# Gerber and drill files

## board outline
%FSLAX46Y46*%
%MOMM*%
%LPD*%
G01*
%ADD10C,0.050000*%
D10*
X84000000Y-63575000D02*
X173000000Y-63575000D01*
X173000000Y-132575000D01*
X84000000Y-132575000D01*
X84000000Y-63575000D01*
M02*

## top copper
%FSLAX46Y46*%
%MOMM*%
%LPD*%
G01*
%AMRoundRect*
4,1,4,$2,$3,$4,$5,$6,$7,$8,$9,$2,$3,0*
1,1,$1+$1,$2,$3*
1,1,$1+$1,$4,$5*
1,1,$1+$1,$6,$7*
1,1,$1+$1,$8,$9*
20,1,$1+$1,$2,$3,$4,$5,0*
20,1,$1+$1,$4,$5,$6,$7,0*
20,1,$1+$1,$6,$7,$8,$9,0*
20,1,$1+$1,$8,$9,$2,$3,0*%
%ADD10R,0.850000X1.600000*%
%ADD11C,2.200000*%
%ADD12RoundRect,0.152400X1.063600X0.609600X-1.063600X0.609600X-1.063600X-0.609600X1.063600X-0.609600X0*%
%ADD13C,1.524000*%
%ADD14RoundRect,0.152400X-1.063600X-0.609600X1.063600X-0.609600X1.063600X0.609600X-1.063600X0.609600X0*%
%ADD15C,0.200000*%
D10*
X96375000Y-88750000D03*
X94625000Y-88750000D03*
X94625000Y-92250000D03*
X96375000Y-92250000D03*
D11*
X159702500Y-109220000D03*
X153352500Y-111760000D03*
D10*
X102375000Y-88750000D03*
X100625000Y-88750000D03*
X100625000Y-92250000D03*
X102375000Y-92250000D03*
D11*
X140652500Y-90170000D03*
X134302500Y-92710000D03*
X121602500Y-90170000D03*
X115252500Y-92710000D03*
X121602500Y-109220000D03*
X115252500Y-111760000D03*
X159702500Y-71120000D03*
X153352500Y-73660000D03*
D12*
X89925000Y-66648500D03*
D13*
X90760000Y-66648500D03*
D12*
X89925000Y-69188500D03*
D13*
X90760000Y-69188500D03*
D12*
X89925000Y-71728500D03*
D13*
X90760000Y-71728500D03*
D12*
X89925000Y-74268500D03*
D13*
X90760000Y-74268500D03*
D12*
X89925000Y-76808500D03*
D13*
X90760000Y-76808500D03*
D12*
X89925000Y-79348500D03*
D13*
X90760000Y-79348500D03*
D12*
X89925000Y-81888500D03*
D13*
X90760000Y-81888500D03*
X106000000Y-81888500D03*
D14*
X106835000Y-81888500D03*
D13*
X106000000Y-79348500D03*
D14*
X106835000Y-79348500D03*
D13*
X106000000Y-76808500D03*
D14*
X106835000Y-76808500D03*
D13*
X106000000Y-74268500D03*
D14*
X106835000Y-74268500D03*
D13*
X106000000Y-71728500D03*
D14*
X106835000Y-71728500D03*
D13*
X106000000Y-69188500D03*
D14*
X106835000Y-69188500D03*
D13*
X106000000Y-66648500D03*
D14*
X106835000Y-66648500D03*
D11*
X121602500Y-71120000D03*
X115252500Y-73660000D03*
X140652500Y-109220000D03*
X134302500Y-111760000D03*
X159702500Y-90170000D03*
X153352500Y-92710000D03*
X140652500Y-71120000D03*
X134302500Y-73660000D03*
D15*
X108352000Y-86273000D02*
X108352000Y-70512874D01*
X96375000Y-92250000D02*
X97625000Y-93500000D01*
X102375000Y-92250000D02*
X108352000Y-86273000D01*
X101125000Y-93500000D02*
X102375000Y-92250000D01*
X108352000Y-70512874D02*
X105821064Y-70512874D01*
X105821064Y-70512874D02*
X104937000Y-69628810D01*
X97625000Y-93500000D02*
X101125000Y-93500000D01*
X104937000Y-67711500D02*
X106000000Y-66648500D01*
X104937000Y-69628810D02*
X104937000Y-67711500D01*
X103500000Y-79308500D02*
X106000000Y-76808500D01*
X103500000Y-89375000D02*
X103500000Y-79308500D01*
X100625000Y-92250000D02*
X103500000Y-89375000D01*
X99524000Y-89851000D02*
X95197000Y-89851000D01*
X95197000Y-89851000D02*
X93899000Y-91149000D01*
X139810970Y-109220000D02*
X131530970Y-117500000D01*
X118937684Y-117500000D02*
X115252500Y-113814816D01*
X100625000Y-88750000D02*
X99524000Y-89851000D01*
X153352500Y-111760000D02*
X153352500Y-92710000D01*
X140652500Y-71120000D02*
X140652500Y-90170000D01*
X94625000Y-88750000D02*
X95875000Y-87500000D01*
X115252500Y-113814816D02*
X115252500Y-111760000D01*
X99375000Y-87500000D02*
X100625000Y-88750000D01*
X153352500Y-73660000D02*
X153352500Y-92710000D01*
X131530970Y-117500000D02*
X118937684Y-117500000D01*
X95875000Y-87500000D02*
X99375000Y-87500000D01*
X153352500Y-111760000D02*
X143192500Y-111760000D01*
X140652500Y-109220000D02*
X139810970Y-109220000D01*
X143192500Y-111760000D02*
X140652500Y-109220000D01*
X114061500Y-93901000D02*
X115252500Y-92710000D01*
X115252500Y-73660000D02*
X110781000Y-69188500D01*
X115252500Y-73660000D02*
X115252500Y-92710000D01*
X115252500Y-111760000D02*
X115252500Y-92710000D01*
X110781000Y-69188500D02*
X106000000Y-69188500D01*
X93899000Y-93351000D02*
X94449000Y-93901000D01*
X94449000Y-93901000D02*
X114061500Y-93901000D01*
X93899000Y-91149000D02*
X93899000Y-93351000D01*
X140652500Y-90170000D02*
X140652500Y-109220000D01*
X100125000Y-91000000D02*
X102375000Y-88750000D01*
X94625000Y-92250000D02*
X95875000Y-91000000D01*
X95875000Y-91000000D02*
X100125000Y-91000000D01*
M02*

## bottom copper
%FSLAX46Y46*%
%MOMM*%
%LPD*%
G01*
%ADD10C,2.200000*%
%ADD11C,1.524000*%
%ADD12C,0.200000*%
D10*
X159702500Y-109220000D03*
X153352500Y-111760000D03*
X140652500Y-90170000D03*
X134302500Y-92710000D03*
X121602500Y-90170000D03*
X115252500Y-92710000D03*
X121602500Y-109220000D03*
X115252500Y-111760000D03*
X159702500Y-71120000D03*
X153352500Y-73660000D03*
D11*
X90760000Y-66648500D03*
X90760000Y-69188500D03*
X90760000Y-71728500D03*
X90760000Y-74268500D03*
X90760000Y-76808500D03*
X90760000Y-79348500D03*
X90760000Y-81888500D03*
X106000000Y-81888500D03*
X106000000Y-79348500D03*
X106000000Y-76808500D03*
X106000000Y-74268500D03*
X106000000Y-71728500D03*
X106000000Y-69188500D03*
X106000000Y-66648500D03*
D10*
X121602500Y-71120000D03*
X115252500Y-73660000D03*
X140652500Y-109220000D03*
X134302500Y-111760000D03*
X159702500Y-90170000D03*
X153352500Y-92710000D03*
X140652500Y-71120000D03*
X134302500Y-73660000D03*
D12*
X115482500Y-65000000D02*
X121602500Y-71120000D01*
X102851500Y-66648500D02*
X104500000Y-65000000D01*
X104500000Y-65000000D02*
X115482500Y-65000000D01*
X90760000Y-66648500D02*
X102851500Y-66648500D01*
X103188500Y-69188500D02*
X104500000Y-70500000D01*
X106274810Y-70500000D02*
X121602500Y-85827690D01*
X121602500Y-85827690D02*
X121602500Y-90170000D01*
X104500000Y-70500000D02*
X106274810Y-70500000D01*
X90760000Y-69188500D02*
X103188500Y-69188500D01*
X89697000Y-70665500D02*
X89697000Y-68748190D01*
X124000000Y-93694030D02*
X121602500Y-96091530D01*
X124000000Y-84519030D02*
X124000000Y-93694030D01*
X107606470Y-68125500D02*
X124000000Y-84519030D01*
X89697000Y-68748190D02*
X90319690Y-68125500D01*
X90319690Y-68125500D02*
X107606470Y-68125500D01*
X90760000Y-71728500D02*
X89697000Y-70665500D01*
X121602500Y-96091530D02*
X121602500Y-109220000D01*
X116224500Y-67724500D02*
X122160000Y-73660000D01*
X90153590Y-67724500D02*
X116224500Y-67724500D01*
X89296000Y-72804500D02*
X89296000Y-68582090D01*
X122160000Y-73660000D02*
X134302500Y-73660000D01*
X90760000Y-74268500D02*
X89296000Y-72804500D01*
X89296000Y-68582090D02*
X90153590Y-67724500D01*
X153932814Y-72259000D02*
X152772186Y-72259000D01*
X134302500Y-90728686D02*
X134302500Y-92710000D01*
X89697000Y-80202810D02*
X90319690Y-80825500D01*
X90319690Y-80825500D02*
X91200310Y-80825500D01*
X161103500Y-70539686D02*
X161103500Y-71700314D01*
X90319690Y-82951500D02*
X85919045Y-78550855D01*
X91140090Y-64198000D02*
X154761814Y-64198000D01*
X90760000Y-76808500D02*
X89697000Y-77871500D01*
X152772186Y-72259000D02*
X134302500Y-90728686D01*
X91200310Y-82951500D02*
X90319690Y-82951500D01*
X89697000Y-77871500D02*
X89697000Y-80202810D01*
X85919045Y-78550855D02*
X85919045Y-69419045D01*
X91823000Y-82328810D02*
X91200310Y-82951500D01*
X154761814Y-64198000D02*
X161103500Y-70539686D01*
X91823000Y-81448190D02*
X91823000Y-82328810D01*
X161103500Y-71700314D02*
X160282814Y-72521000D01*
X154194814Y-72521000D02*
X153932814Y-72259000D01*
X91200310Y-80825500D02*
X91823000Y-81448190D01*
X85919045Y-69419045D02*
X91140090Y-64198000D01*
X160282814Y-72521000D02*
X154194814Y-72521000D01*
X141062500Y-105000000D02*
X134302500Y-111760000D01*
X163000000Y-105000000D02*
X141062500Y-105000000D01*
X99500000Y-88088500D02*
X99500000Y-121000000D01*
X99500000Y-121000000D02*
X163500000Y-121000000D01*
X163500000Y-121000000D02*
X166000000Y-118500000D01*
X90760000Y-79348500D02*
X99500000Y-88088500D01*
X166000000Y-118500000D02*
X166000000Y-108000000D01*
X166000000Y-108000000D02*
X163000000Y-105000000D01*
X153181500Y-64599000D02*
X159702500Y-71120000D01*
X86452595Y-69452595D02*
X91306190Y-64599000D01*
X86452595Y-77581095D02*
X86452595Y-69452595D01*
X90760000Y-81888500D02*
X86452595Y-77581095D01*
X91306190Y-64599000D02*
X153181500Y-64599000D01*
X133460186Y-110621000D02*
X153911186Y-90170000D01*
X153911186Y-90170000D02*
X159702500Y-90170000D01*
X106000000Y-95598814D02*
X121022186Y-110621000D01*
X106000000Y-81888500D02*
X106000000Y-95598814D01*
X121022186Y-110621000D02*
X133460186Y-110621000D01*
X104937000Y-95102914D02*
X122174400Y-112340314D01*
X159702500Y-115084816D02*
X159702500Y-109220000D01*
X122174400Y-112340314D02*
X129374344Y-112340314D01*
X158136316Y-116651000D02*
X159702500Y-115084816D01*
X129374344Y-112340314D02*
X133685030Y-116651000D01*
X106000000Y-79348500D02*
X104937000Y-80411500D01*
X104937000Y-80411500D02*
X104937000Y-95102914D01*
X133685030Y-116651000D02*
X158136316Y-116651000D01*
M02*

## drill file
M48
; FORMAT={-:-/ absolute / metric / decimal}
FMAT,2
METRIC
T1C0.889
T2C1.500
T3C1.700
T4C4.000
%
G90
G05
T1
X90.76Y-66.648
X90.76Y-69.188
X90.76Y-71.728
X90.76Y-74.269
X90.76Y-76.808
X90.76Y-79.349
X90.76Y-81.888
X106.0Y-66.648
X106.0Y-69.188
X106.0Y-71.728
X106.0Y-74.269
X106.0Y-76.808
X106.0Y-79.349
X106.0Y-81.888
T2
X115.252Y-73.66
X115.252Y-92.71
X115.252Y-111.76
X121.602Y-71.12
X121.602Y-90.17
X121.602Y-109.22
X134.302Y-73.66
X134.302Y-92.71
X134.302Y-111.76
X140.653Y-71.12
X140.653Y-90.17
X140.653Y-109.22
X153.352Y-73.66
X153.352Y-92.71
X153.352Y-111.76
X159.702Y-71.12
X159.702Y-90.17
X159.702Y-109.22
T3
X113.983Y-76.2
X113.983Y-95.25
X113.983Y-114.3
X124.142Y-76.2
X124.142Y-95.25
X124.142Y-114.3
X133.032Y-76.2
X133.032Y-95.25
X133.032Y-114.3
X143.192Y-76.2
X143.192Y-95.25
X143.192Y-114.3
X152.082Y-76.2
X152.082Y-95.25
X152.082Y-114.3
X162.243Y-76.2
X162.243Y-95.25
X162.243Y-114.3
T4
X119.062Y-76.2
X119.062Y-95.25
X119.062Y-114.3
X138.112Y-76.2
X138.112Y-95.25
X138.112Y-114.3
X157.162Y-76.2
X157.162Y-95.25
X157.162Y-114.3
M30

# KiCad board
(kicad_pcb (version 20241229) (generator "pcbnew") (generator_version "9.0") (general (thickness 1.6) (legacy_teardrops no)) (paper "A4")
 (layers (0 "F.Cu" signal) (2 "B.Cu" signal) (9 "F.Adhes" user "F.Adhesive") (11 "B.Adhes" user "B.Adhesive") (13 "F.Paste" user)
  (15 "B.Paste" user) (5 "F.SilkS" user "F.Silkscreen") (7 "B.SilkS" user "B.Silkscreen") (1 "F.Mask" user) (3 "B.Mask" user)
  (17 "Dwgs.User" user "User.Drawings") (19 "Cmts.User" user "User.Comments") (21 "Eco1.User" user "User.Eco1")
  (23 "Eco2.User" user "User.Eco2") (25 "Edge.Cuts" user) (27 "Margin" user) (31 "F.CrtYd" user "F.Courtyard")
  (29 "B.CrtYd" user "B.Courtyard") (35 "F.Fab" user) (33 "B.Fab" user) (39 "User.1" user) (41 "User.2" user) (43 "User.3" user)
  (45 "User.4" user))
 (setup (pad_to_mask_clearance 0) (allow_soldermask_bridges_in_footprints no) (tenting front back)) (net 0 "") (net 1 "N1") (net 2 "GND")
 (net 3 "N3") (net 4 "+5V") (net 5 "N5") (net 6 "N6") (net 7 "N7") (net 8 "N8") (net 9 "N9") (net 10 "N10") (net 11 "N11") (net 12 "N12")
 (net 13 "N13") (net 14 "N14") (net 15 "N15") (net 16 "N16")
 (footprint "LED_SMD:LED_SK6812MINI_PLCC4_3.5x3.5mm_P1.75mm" (layer "F.Cu") (at 95.5 90.5 -90)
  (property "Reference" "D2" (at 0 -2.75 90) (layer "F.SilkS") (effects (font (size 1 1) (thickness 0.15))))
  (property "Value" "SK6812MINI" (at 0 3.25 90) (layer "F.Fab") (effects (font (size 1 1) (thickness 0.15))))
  (pad "1" smd rect (at -1.75 -0.875 270) (size 1.6 0.85) (layers "F.Cu" "F.Mask" "F.Paste") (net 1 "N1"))
  (pad "2" smd rect (at -1.75 0.875 270) (size 1.6 0.85) (layers "F.Cu" "F.Mask" "F.Paste") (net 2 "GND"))
  (pad "3" smd rect (at 1.75 0.875 270) (size 1.6 0.85) (layers "F.Cu" "F.Mask" "F.Paste") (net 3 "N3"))
  (pad "4" smd rect (at 1.75 -0.875 270) (size 1.6 0.85) (layers "F.Cu" "F.Mask" "F.Paste") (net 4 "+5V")))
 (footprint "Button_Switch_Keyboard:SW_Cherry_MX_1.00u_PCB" (layer "F.Cu") (at 159.7025 109.22)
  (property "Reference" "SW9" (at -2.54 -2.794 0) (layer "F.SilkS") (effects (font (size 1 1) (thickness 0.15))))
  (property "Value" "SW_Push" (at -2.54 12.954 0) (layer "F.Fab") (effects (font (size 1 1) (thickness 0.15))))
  (pad "" np_thru_hole circle (at -7.62 5.08) (size 1.7 1.7) (drill 1.7) (layers "*.Cu" "*.Mask"))
  (pad "" np_thru_hole circle (at -2.54 5.08) (size 4 4) (drill 4) (layers "*.Cu" "*.Mask"))
  (pad "" np_thru_hole circle (at 2.54 5.08) (size 1.7 1.7) (drill 1.7) (layers "*.Cu" "*.Mask"))
  (pad "1" thru_hole circle (at 0 0) (size 2.2 2.2) (drill 1.5) (layers "*.Cu" "*.Mask") (remove_unused_layers no) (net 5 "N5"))
  (pad "2" thru_hole circle (at -6.35 2.54) (size 2.2 2.2) (drill 1.5) (layers "*.Cu" "*.Mask") (remove_unused_layers no) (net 2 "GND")))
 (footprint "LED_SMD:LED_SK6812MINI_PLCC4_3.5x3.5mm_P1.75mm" (layer "F.Cu") (at 101.5 90.5 -90)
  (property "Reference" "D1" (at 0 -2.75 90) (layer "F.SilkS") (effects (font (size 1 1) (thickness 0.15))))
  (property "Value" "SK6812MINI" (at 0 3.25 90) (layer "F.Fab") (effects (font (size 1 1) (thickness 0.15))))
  (pad "1" smd rect (at -1.75 -0.875 270) (size 1.6 0.85) (layers "F.Cu" "F.Mask" "F.Paste") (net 3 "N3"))
  (pad "2" smd rect (at -1.75 0.875 270) (size 1.6 0.85) (layers "F.Cu" "F.Mask" "F.Paste") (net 2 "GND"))
  (pad "3" smd rect (at 1.75 0.875 270) (size 1.6 0.85) (layers "F.Cu" "F.Mask" "F.Paste") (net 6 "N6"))
  (pad "4" smd rect (at 1.75 -0.875 270) (size 1.6 0.85) (layers "F.Cu" "F.Mask" "F.Paste") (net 4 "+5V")))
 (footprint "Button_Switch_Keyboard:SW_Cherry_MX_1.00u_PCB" (layer "F.Cu") (at 140.6525 90.17)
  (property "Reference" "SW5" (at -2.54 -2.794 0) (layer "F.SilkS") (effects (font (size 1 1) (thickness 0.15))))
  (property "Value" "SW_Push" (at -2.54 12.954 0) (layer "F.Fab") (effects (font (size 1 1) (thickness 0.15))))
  (pad "" np_thru_hole circle (at -7.62 5.08) (size 1.7 1.7) (drill 1.7) (layers "*.Cu" "*.Mask"))
  (pad "" np_thru_hole circle (at -2.54 5.08) (size 4 4) (drill 4) (layers "*.Cu" "*.Mask"))
  (pad "" np_thru_hole circle (at 2.54 5.08) (size 1.7 1.7) (drill 1.7) (layers "*.Cu" "*.Mask"))
  (pad "1" thru_hole circle (at 0 0) (size 2.2 2.2) (drill 1.5) (layers "*.Cu" "*.Mask") (remove_unused_layers no) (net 2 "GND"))
  (pad "2" thru_hole circle (at -6.35 2.54) (size 2.2 2.2) (drill 1.5) (layers "*.Cu" "*.Mask") (remove_unused_layers no) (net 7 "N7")))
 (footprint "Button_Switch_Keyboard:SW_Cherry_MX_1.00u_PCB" (layer "F.Cu") (at 121.6025 90.17)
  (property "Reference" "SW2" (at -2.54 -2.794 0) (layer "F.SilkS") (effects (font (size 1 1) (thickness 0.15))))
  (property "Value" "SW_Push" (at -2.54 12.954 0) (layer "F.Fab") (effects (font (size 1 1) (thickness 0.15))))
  (pad "" np_thru_hole circle (at -7.62 5.08) (size 1.7 1.7) (drill 1.7) (layers "*.Cu" "*.Mask"))
  (pad "" np_thru_hole circle (at -2.54 5.08) (size 4 4) (drill 4) (layers "*.Cu" "*.Mask"))
  (pad "" np_thru_hole circle (at 2.54 5.08) (size 1.7 1.7) (drill 1.7) (layers "*.Cu" "*.Mask"))
  (pad "1" thru_hole circle (at 0 0) (size 2.2 2.2) (drill 1.5) (layers "*.Cu" "*.Mask") (remove_unused_layers no) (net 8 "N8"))
  (pad "2" thru_hole circle (at -6.35 2.54) (size 2.2 2.2) (drill 1.5) (layers "*.Cu" "*.Mask") (remove_unused_layers no) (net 2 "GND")))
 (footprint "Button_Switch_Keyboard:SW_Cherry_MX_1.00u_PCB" (layer "F.Cu") (at 121.6025 109.22)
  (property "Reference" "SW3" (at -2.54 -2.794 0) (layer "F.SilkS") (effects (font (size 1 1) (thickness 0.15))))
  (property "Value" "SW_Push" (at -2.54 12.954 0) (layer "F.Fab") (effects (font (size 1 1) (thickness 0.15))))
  (pad "" np_thru_hole circle (at -7.62 5.08) (size 1.7 1.7) (drill 1.7) (layers "*.Cu" "*.Mask"))
  (pad "" np_thru_hole circle (at -2.54 5.08) (size 4 4) (drill 4) (layers "*.Cu" "*.Mask"))
  (pad "" np_thru_hole circle (at 2.54 5.08) (size 1.7 1.7) (drill 1.7) (layers "*.Cu" "*.Mask"))
  (pad "1" thru_hole circle (at 0 0) (size 2.2 2.2) (drill 1.5) (layers "*.Cu" "*.Mask") (remove_unused_layers no) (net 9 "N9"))
  (pad "2" thru_hole circle (at -6.35 2.54) (size 2.2 2.2) (drill 1.5) (layers "*.Cu" "*.Mask") (remove_unused_layers no) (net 2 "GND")))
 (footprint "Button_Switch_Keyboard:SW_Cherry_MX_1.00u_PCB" (layer "F.Cu") (at 159.7025 71.12)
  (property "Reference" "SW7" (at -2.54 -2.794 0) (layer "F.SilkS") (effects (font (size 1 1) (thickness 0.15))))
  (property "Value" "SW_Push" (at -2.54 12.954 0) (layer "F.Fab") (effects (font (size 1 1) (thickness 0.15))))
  (pad "" np_thru_hole circle (at -7.62 5.08) (size 1.7 1.7) (drill 1.7) (layers "*.Cu" "*.Mask"))
  (pad "" np_thru_hole circle (at -2.54 5.08) (size 4 4) (drill 4) (layers "*.Cu" "*.Mask"))
  (pad "" np_thru_hole circle (at 2.54 5.08) (size 1.7 1.7) (drill 1.7) (layers "*.Cu" "*.Mask"))
  (pad "1" thru_hole circle (at 0 0) (size 2.2 2.2) (drill 1.5) (layers "*.Cu" "*.Mask") (remove_unused_layers no) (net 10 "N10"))
  (pad "2" thru_hole circle (at -6.35 2.54) (size 2.2 2.2) (drill 1.5) (layers "*.Cu" "*.Mask") (remove_unused_layers no) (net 2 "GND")))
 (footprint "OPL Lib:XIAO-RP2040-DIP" (layer "F.Cu") (at 98.38 74.2685)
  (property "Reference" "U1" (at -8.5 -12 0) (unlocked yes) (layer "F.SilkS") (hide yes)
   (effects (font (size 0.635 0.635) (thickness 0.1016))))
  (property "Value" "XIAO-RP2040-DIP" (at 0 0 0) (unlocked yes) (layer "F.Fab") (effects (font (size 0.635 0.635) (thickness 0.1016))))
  (pad "1" smd roundrect (at -8.455 -7.62 180) (size 2.432 1.524) (layers "F.Cu" "F.Mask") (roundrect_rratio 0.1) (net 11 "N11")
   (thermal_bridge_angle 45))
  (pad "1" thru_hole circle (at -7.62 -7.62 180) (size 1.524 1.524) (drill 0.889) (layers "*.Cu" "*.Mask") (remove_unused_layers no)
   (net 11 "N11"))
  (pad "2" smd roundrect (at -8.455 -5.08 180) (size 2.432 1.524) (layers "F.Cu" "F.Mask") (roundrect_rratio 0.1) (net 8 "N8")
   (thermal_bridge_angle 45))
  (pad "2" thru_hole circle (at -7.62 -5.08 180) (size 1.524 1.524) (drill 0.889) (layers "*.Cu" "*.Mask") (remove_unused_layers no)
   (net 8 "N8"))
  (pad "3" smd roundrect (at -8.455 -2.54 180) (size 2.432 1.524) (layers "F.Cu" "F.Mask") (roundrect_rratio 0.1) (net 9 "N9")
   (thermal_bridge_angle 45))
  (pad "3" thru_hole circle (at -7.62 -2.54 180) (size 1.524 1.524) (drill 0.889) (layers "*.Cu" "*.Mask") (remove_unused_layers no)
   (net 9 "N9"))
  (pad "4" smd roundrect (at -8.455 0 180) (size 2.432 1.524) (layers "F.Cu" "F.Mask") (roundrect_rratio 0.1) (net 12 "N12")
   (thermal_bridge_angle 45))
  (pad "4" thru_hole circle (at -7.62 0 180) (size 1.524 1.524) (drill 0.889) (layers "*.Cu" "*.Mask") (remove_unused_layers no)
   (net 12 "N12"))
  (pad "5" smd roundrect (at -8.455 2.54 180) (size 2.432 1.524) (layers "F.Cu" "F.Mask") (roundrect_rratio 0.1) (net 7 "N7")
   (thermal_bridge_angle 45))
  (pad "5" thru_hole circle (at -7.62 2.54 180) (size 1.524 1.524) (drill 0.889) (layers "*.Cu" "*.Mask") (remove_unused_layers no)
   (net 7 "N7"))
  (pad "6" smd roundrect (at -8.455 5.08 180) (size 2.432 1.524) (layers "F.Cu" "F.Mask") (roundrect_rratio 0.1) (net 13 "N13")
   (thermal_bridge_angle 45))
  (pad "6" thru_hole circle (at -7.62 5.08 180) (size 1.524 1.524) (drill 0.889) (layers "*.Cu" "*.Mask") (remove_unused_layers no)
   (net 13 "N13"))
  (pad "7" smd roundrect (at -8.455 7.62 180) (size 2.432 1.524) (layers "F.Cu" "F.Mask") (roundrect_rratio 0.1) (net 10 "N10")
   (thermal_bridge_angle 45))
  (pad "7" thru_hole circle (at -7.62 7.62 180) (size 1.524 1.524) (drill 0.889) (layers "*.Cu" "*.Mask") (remove_unused_layers no)
   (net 10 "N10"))
  (pad "8" thru_hole circle (at 7.62 7.62) (size 1.524 1.524) (drill 0.889) (layers "*.Cu" "*.Mask") (remove_unused_layers no)
   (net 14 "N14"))
  (pad "8" smd roundrect (at 8.455 7.62) (size 2.432 1.524) (layers "F.Cu" "F.Mask") (roundrect_rratio 0.1) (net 14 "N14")
   (thermal_bridge_angle 45))
  (pad "9" thru_hole circle (at 7.62 5.08) (size 1.524 1.524) (drill 0.889) (layers "*.Cu" "*.Mask") (remove_unused_layers no) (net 5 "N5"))
  (pad "9" smd roundrect (at 8.455 5.08) (size 2.432 1.524) (layers "F.Cu" "F.Mask") (roundrect_rratio 0.1) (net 5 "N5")
   (thermal_bridge_angle 45))
  (pad "10" thru_hole circle (at 7.62 2.54) (size 1.524 1.524) (drill 0.889) (layers "*.Cu" "*.Mask") (remove_unused_layers no) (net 6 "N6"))
  (pad "10" smd roundrect (at 8.455 2.54) (size 2.432 1.524) (layers "F.Cu" "F.Mask") (roundrect_rratio 0.1) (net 6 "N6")
   (thermal_bridge_angle 45))
  (pad "11" thru_hole circle (at 7.62 0) (size 1.524 1.524) (drill 0.889) (layers "*.Cu" "*.Mask") (remove_unused_layers no) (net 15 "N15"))
  (pad "11" smd roundrect (at 8.455 0) (size 2.432 1.524) (layers "F.Cu" "F.Mask") (roundrect_rratio 0.1) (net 15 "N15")
   (thermal_bridge_angle 45))
  (pad "12" thru_hole circle (at 7.62 -2.54) (size 1.524 1.524) (drill 0.889) (layers "*.Cu" "*.Mask") (remove_unused_layers no)
   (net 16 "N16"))
  (pad "12" smd roundrect (at 8.455 -2.54) (size 2.432 1.524) (layers "F.Cu" "F.Mask") (roundrect_rratio 0.1) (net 16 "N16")
   (thermal_bridge_angle 45))
  (pad "13" thru_hole circle (at 7.62 -5.08) (size 1.524 1.524) (drill 0.889) (layers "*.Cu" "*.Mask") (remove_unused_layers no)
   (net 2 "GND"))
  (pad "13" smd roundrect (at 8.455 -5.08) (size 2.432 1.524) (layers "F.Cu" "F.Mask") (roundrect_rratio 0.1) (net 2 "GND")
   (thermal_bridge_angle 45))
  (pad "14" thru_hole circle (at 7.62 -7.62) (size 1.524 1.524) (drill 0.889) (layers "*.Cu" "*.Mask") (remove_unused_layers no)
   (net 4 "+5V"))
  (pad "14" smd roundrect (at 8.455 -7.62) (size 2.432 1.524) (layers "F.Cu" "F.Mask") (roundrect_rratio 0.1) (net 4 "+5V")
   (thermal_bridge_angle 45)))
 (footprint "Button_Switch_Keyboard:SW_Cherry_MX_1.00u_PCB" (layer "F.Cu") (at 121.6025 71.12)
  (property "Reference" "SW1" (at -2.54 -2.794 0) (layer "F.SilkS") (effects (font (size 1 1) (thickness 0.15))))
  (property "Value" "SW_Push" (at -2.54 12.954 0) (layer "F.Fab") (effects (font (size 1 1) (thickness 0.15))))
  (pad "" np_thru_hole circle (at -7.62 5.08) (size 1.7 1.7) (drill 1.7) (layers "*.Cu" "*.Mask"))
  (pad "" np_thru_hole circle (at -2.54 5.08) (size 4 4) (drill 4) (layers "*.Cu" "*.Mask"))
  (pad "" np_thru_hole circle (at 2.54 5.08) (size 1.7 1.7) (drill 1.7) (layers "*.Cu" "*.Mask"))
  (pad "1" thru_hole circle (at 0 0) (size 2.2 2.2) (drill 1.5) (layers "*.Cu" "*.Mask") (remove_unused_layers no) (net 11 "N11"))
  (pad "2" thru_hole circle (at -6.35 2.54) (size 2.2 2.2) (drill 1.5) (layers "*.Cu" "*.Mask") (remove_unused_layers no) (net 2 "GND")))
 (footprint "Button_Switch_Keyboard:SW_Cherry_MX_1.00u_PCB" (layer "F.Cu") (at 140.6525 109.22)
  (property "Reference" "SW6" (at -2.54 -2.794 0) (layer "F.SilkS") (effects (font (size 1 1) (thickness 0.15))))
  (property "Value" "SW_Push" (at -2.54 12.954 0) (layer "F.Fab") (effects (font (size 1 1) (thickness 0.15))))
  (pad "" np_thru_hole circle (at -7.62 5.08) (size 1.7 1.7) (drill 1.7) (layers "*.Cu" "*.Mask"))
  (pad "" np_thru_hole circle (at -2.54 5.08) (size 4 4) (drill 4) (layers "*.Cu" "*.Mask"))
  (pad "" np_thru_hole circle (at 2.54 5.08) (size 1.7 1.7) (drill 1.7) (layers "*.Cu" "*.Mask"))
  (pad "1" thru_hole circle (at 0 0) (size 2.2 2.2) (drill 1.5) (layers "*.Cu" "*.Mask") (remove_unused_layers no) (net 2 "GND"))
  (pad "2" thru_hole circle (at -6.35 2.54) (size 2.2 2.2) (drill 1.5) (layers "*.Cu" "*.Mask") (remove_unused_layers no) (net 13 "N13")))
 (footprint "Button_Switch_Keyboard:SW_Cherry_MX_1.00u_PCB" (layer "F.Cu") (at 159.7025 90.17)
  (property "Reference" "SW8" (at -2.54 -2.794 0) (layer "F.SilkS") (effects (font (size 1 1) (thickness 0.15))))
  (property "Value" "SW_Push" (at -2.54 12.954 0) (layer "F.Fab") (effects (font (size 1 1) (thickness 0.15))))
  (pad "" np_thru_hole circle (at -7.62 5.08) (size 1.7 1.7) (drill 1.7) (layers "*.Cu" "*.Mask"))
  (pad "" np_thru_hole circle (at -2.54 5.08) (size 4 4) (drill 4) (layers "*.Cu" "*.Mask"))
  (pad "" np_thru_hole circle (at 2.54 5.08) (size 1.7 1.7) (drill 1.7) (layers "*.Cu" "*.Mask"))
  (pad "1" thru_hole circle (at 0 0) (size 2.2 2.2) (drill 1.5) (layers "*.Cu" "*.Mask") (remove_unused_layers no) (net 14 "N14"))
  (pad "2" thru_hole circle (at -6.35 2.54) (size 2.2 2.2) (drill 1.5) (layers "*.Cu" "*.Mask") (remove_unused_layers no) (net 2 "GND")))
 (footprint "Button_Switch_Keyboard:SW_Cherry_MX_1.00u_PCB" (layer "F.Cu") (at 140.6525 71.12)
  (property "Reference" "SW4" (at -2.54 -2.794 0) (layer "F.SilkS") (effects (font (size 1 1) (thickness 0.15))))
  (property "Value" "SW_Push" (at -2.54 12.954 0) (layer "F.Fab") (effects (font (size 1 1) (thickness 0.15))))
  (pad "" np_thru_hole circle (at -7.62 5.08) (size 1.7 1.7) (drill 1.7) (layers "*.Cu" "*.Mask"))
  (pad "" np_thru_hole circle (at -2.54 5.08) (size 4 4) (drill 4) (layers "*.Cu" "*.Mask"))
  (pad "" np_thru_hole circle (at 2.54 5.08) (size 1.7 1.7) (drill 1.7) (layers "*.Cu" "*.Mask"))
  (pad "1" thru_hole circle (at 0 0) (size 2.2 2.2) (drill 1.5) (layers "*.Cu" "*.Mask") (remove_unused_layers no) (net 2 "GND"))
  (pad "2" thru_hole circle (at -6.35 2.54) (size 2.2 2.2) (drill 1.5) (layers "*.Cu" "*.Mask") (remove_unused_layers no) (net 12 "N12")))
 (gr_rect (start 84 63.575) (end 173 132.575) (stroke (width 0.05) (type default)) (fill no) (layer "Edge.Cuts"))
 (segment (start 108.352 86.273) (end 108.352 70.512874) (width 0.2) (layer "F.Cu") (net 4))
 (segment (start 96.375 92.25) (end 97.625 93.5) (width 0.2) (layer "F.Cu") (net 4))
 (segment (start 102.375 92.25) (end 108.352 86.273) (width 0.2) (layer "F.Cu") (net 4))
 (segment (start 101.125 93.5) (end 102.375 92.25) (width 0.2) (layer "F.Cu") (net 4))
 (segment (start 108.352 70.512874) (end 105.821064 70.512874) (width 0.2) (layer "F.Cu") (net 4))
 (segment (start 105.821064 70.512874) (end 104.937 69.62881) (width 0.2) (layer "F.Cu") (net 4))
 (segment (start 97.625 93.5) (end 101.125 93.5) (width 0.2) (layer "F.Cu") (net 4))
 (segment (start 104.937 67.7115) (end 106 66.6485) (width 0.2) (layer "F.Cu") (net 4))
 (segment (start 104.937 69.62881) (end 104.937 67.7115) (width 0.2) (layer "F.Cu") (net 4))
 (segment (start 103.5 79.3085) (end 106 76.8085) (width 0.2) (layer "F.Cu") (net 6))
 (segment (start 103.5 89.375) (end 103.5 79.3085) (width 0.2) (layer "F.Cu") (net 6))
 (segment (start 100.625 92.25) (end 103.5 89.375) (width 0.2) (layer "F.Cu") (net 6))
 (segment (start 99.524 89.851) (end 95.197 89.851) (width 0.2) (layer "F.Cu") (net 2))
 (segment (start 95.197 89.851) (end 93.899 91.149) (width 0.2) (layer "F.Cu") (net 2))
 (segment (start 139.81097 109.22) (end 131.53097 117.5) (width 0.2) (layer "F.Cu") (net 2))
 (segment (start 118.937684 117.5) (end 115.2525 113.814816) (width 0.2) (layer "F.Cu") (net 2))
 (segment (start 100.625 88.75) (end 99.524 89.851) (width 0.2) (layer "F.Cu") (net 2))
 (segment (start 153.3525 111.76) (end 153.3525 92.71) (width 0.2) (layer "F.Cu") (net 2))
 (segment (start 140.6525 71.12) (end 140.6525 90.17) (width 0.2) (layer "F.Cu") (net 2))
 (segment (start 94.625 88.75) (end 95.875 87.5) (width 0.2) (layer "F.Cu") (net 2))
 (segment (start 115.2525 113.814816) (end 115.2525 111.76) (width 0.2) (layer "F.Cu") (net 2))
 (segment (start 99.375 87.5) (end 100.625 88.75) (width 0.2) (layer "F.Cu") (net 2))
 (segment (start 153.3525 73.66) (end 153.3525 92.71) (width 0.2) (layer "F.Cu") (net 2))
 (segment (start 131.53097 117.5) (end 118.937684 117.5) (width 0.2) (layer "F.Cu") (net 2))
 (segment (start 95.875 87.5) (end 99.375 87.5) (width 0.2) (layer "F.Cu") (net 2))
 (segment (start 153.3525 111.76) (end 143.1925 111.76) (width 0.2) (layer "F.Cu") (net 2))
 (segment (start 140.6525 109.22) (end 139.81097 109.22) (width 0.2) (layer "F.Cu") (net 2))
 (segment (start 143.1925 111.76) (end 140.6525 109.22) (width 0.2) (layer "F.Cu") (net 2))
 (segment (start 114.0615 93.901) (end 115.2525 92.71) (width 0.2) (layer "F.Cu") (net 2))
 (segment (start 115.2525 73.66) (end 110.781 69.1885) (width 0.2) (layer "F.Cu") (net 2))
 (segment (start 115.2525 73.66) (end 115.2525 92.71) (width 0.2) (layer "F.Cu") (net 2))
 (segment (start 115.2525 111.76) (end 115.2525 92.71) (width 0.2) (layer "F.Cu") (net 2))
 (segment (start 110.781 69.1885) (end 106 69.1885) (width 0.2) (layer "F.Cu") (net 2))
 (segment (start 93.899 93.351) (end 94.449 93.901) (width 0.2) (layer "F.Cu") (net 2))
 (segment (start 94.449 93.901) (end 114.0615 93.901) (width 0.2) (layer "F.Cu") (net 2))
 (segment (start 93.899 91.149) (end 93.899 93.351) (width 0.2) (layer "F.Cu") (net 2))
 (segment (start 140.6525 90.17) (end 140.6525 109.22) (width 0.2) (layer "F.Cu") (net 2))
 (segment (start 100.125 91) (end 102.375 88.75) (width 0.2) (layer "F.Cu") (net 3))
 (segment (start 94.625 92.25) (end 95.875 91) (width 0.2) (layer "F.Cu") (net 3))
 (segment (start 95.875 91) (end 100.125 91) (width 0.2) (layer "F.Cu") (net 3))
 (segment (start 115.4825 65) (end 121.6025 71.12) (width 0.2) (layer "B.Cu") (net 11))
 (segment (start 102.8515 66.6485) (end 104.5 65) (width 0.2) (layer "B.Cu") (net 11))
 (segment (start 104.5 65) (end 115.4825 65) (width 0.2) (layer "B.Cu") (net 11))
 (segment (start 90.76 66.6485) (end 102.8515 66.6485) (width 0.2) (layer "B.Cu") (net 11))
 (segment (start 103.1885 69.1885) (end 104.5 70.5) (width 0.2) (layer "B.Cu") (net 8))
 (segment (start 106.27481 70.5) (end 121.6025 85.82769) (width 0.2) (layer "B.Cu") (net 8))
 (segment (start 121.6025 85.82769) (end 121.6025 90.17) (width 0.2) (layer "B.Cu") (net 8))
 (segment (start 104.5 70.5) (end 106.27481 70.5) (width 0.2) (layer "B.Cu") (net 8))
 (segment (start 90.76 69.1885) (end 103.1885 69.1885) (width 0.2) (layer "B.Cu") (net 8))
 (segment (start 89.697 70.6655) (end 89.697 68.74819) (width 0.2) (layer "B.Cu") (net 9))
 (segment (start 124 93.69403) (end 121.6025 96.09153) (width 0.2) (layer "B.Cu") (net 9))
 (segment (start 124 84.51903) (end 124 93.69403) (width 0.2) (layer "B.Cu") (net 9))
 (segment (start 107.60647 68.1255) (end 124 84.51903) (width 0.2) (layer "B.Cu") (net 9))
 (segment (start 89.697 68.74819) (end 90.31969 68.1255) (width 0.2) (layer "B.Cu") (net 9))
 (segment (start 90.31969 68.1255) (end 107.60647 68.1255) (width 0.2) (layer "B.Cu") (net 9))
 (segment (start 90.76 71.7285) (end 89.697 70.6655) (width 0.2) (layer "B.Cu") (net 9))
 (segment (start 121.6025 96.09153) (end 121.6025 109.22) (width 0.2) (layer "B.Cu") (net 9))
 (segment (start 116.2245 67.7245) (end 122.16 73.66) (width 0.2) (layer "B.Cu") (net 12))
 (segment (start 90.15359 67.7245) (end 116.2245 67.7245) (width 0.2) (layer "B.Cu") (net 12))
 (segment (start 89.296 72.8045) (end 89.296 68.58209) (width 0.2) (layer "B.Cu") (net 12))
 (segment (start 122.16 73.66) (end 134.3025 73.66) (width 0.2) (layer "B.Cu") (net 12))
 (segment (start 90.76 74.2685) (end 89.296 72.8045) (width 0.2) (layer "B.Cu") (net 12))
 (segment (start 89.296 68.58209) (end 90.15359 67.7245) (width 0.2) (layer "B.Cu") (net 12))
 (segment (start 153.932814 72.259) (end 152.772186 72.259) (width 0.2) (layer "B.Cu") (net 7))
 (segment (start 134.3025 90.728686) (end 134.3025 92.71) (width 0.2) (layer "B.Cu") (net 7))
 (segment (start 89.697 80.20281) (end 90.31969 80.8255) (width 0.2) (layer "B.Cu") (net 7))
 (segment (start 90.31969 80.8255) (end 91.20031 80.8255) (width 0.2) (layer "B.Cu") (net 7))
 (segment (start 161.1035 70.539686) (end 161.1035 71.700314) (width 0.2) (layer "B.Cu") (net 7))
 (segment (start 90.31969 82.9515) (end 85.919045 78.550855) (width 0.2) (layer "B.Cu") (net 7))
 (segment (start 91.14009 64.198) (end 154.761814 64.198) (width 0.2) (layer "B.Cu") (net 7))
 (segment (start 90.76 76.8085) (end 89.697 77.8715) (width 0.2) (layer "B.Cu") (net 7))
 (segment (start 152.772186 72.259) (end 134.3025 90.728686) (width 0.2) (layer "B.Cu") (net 7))
 (segment (start 91.20031 82.9515) (end 90.31969 82.9515) (width 0.2) (layer "B.Cu") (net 7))
 (segment (start 89.697 77.8715) (end 89.697 80.20281) (width 0.2) (layer "B.Cu") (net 7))
 (segment (start 85.919045 78.550855) (end 85.919045 69.419045) (width 0.2) (layer "B.Cu") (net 7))
 (segment (start 91.823 82.32881) (end 91.20031 82.9515) (width 0.2) (layer "B.Cu") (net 7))
 (segment (start 154.761814 64.198) (end 161.1035 70.539686) (width 0.2) (layer "B.Cu") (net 7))
 (segment (start 91.823 81.44819) (end 91.823 82.32881) (width 0.2) (layer "B.Cu") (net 7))
 (segment (start 161.1035 71.700314) (end 160.282814 72.521) (width 0.2) (layer "B.Cu") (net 7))
 (segment (start 154.194814 72.521) (end 153.932814 72.259) (width 0.2) (layer "B.Cu") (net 7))
 (segment (start 91.20031 80.8255) (end 91.823 81.44819) (width 0.2) (layer "B.Cu") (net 7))
 (segment (start 85.919045 69.419045) (end 91.14009 64.198) (width 0.2) (layer "B.Cu") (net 7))
 (segment (start 160.282814 72.521) (end 154.194814 72.521) (width 0.2) (layer "B.Cu") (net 7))
 (segment (start 141.0625 105) (end 134.3025 111.76) (width 0.2) (layer "B.Cu") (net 13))
 (segment (start 163 105) (end 141.0625 105) (width 0.2) (layer "B.Cu") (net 13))
 (segment (start 99.5 88.0885) (end 99.5 121) (width 0.2) (layer "B.Cu") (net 13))
 (segment (start 99.5 121) (end 163.5 121) (width 0.2) (layer "B.Cu") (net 13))
 (segment (start 163.5 121) (end 166 118.5) (width 0.2) (layer "B.Cu") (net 13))
 (segment (start 90.76 79.3485) (end 99.5 88.0885) (width 0.2) (layer "B.Cu") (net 13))
 (segment (start 166 118.5) (end 166 108) (width 0.2) (layer "B.Cu") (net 13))
 (segment (start 166 108) (end 163 105) (width 0.2) (layer "B.Cu") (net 13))
 (segment (start 153.1815 64.599) (end 159.7025 71.12) (width 0.2) (layer "B.Cu") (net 10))
 (segment (start 86.452595 69.452595) (end 91.30619 64.599) (width 0.2) (layer "B.Cu") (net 10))
 (segment (start 86.452595 77.581095) (end 86.452595 69.452595) (width 0.2) (layer "B.Cu") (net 10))
 (segment (start 90.76 81.8885) (end 86.452595 77.581095) (width 0.2) (layer "B.Cu") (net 10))
 (segment (start 91.30619 64.599) (end 153.1815 64.599) (width 0.2) (layer "B.Cu") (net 10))
 (segment (start 133.460186 110.621) (end 153.911186 90.17) (width 0.2) (layer "B.Cu") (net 14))
 (segment (start 153.911186 90.17) (end 159.7025 90.17) (width 0.2) (layer "B.Cu") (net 14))
 (segment (start 106 95.598814) (end 121.022186 110.621) (width 0.2) (layer "B.Cu") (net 14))
 (segment (start 106 81.8885) (end 106 95.598814) (width 0.2) (layer "B.Cu") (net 14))
 (segment (start 121.022186 110.621) (end 133.460186 110.621) (width 0.2) (layer "B.Cu") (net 14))
 (segment (start 104.937 95.102914) (end 122.1744 112.340314) (width 0.2) (layer "B.Cu") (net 5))
 (segment (start 159.7025 115.084816) (end 159.7025 109.22) (width 0.2) (layer "B.Cu") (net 5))
 (segment (start 122.1744 112.340314) (end 129.374344 112.340314) (width 0.2) (layer "B.Cu") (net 5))
 (segment (start 158.136316 116.651) (end 159.7025 115.084816) (width 0.2) (layer "B.Cu") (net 5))
 (segment (start 129.374344 112.340314) (end 133.68503 116.651) (width 0.2) (layer "B.Cu") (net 5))
 (segment (start 106 79.3485) (end 104.937 80.4115) (width 0.2) (layer "B.Cu") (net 5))
 (segment (start 104.937 80.4115) (end 104.937 95.102914) (width 0.2) (layer "B.Cu") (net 5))
 (segment (start 133.68503 116.651) (end 158.136316 116.651) (width 0.2) (layer "B.Cu") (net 5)))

